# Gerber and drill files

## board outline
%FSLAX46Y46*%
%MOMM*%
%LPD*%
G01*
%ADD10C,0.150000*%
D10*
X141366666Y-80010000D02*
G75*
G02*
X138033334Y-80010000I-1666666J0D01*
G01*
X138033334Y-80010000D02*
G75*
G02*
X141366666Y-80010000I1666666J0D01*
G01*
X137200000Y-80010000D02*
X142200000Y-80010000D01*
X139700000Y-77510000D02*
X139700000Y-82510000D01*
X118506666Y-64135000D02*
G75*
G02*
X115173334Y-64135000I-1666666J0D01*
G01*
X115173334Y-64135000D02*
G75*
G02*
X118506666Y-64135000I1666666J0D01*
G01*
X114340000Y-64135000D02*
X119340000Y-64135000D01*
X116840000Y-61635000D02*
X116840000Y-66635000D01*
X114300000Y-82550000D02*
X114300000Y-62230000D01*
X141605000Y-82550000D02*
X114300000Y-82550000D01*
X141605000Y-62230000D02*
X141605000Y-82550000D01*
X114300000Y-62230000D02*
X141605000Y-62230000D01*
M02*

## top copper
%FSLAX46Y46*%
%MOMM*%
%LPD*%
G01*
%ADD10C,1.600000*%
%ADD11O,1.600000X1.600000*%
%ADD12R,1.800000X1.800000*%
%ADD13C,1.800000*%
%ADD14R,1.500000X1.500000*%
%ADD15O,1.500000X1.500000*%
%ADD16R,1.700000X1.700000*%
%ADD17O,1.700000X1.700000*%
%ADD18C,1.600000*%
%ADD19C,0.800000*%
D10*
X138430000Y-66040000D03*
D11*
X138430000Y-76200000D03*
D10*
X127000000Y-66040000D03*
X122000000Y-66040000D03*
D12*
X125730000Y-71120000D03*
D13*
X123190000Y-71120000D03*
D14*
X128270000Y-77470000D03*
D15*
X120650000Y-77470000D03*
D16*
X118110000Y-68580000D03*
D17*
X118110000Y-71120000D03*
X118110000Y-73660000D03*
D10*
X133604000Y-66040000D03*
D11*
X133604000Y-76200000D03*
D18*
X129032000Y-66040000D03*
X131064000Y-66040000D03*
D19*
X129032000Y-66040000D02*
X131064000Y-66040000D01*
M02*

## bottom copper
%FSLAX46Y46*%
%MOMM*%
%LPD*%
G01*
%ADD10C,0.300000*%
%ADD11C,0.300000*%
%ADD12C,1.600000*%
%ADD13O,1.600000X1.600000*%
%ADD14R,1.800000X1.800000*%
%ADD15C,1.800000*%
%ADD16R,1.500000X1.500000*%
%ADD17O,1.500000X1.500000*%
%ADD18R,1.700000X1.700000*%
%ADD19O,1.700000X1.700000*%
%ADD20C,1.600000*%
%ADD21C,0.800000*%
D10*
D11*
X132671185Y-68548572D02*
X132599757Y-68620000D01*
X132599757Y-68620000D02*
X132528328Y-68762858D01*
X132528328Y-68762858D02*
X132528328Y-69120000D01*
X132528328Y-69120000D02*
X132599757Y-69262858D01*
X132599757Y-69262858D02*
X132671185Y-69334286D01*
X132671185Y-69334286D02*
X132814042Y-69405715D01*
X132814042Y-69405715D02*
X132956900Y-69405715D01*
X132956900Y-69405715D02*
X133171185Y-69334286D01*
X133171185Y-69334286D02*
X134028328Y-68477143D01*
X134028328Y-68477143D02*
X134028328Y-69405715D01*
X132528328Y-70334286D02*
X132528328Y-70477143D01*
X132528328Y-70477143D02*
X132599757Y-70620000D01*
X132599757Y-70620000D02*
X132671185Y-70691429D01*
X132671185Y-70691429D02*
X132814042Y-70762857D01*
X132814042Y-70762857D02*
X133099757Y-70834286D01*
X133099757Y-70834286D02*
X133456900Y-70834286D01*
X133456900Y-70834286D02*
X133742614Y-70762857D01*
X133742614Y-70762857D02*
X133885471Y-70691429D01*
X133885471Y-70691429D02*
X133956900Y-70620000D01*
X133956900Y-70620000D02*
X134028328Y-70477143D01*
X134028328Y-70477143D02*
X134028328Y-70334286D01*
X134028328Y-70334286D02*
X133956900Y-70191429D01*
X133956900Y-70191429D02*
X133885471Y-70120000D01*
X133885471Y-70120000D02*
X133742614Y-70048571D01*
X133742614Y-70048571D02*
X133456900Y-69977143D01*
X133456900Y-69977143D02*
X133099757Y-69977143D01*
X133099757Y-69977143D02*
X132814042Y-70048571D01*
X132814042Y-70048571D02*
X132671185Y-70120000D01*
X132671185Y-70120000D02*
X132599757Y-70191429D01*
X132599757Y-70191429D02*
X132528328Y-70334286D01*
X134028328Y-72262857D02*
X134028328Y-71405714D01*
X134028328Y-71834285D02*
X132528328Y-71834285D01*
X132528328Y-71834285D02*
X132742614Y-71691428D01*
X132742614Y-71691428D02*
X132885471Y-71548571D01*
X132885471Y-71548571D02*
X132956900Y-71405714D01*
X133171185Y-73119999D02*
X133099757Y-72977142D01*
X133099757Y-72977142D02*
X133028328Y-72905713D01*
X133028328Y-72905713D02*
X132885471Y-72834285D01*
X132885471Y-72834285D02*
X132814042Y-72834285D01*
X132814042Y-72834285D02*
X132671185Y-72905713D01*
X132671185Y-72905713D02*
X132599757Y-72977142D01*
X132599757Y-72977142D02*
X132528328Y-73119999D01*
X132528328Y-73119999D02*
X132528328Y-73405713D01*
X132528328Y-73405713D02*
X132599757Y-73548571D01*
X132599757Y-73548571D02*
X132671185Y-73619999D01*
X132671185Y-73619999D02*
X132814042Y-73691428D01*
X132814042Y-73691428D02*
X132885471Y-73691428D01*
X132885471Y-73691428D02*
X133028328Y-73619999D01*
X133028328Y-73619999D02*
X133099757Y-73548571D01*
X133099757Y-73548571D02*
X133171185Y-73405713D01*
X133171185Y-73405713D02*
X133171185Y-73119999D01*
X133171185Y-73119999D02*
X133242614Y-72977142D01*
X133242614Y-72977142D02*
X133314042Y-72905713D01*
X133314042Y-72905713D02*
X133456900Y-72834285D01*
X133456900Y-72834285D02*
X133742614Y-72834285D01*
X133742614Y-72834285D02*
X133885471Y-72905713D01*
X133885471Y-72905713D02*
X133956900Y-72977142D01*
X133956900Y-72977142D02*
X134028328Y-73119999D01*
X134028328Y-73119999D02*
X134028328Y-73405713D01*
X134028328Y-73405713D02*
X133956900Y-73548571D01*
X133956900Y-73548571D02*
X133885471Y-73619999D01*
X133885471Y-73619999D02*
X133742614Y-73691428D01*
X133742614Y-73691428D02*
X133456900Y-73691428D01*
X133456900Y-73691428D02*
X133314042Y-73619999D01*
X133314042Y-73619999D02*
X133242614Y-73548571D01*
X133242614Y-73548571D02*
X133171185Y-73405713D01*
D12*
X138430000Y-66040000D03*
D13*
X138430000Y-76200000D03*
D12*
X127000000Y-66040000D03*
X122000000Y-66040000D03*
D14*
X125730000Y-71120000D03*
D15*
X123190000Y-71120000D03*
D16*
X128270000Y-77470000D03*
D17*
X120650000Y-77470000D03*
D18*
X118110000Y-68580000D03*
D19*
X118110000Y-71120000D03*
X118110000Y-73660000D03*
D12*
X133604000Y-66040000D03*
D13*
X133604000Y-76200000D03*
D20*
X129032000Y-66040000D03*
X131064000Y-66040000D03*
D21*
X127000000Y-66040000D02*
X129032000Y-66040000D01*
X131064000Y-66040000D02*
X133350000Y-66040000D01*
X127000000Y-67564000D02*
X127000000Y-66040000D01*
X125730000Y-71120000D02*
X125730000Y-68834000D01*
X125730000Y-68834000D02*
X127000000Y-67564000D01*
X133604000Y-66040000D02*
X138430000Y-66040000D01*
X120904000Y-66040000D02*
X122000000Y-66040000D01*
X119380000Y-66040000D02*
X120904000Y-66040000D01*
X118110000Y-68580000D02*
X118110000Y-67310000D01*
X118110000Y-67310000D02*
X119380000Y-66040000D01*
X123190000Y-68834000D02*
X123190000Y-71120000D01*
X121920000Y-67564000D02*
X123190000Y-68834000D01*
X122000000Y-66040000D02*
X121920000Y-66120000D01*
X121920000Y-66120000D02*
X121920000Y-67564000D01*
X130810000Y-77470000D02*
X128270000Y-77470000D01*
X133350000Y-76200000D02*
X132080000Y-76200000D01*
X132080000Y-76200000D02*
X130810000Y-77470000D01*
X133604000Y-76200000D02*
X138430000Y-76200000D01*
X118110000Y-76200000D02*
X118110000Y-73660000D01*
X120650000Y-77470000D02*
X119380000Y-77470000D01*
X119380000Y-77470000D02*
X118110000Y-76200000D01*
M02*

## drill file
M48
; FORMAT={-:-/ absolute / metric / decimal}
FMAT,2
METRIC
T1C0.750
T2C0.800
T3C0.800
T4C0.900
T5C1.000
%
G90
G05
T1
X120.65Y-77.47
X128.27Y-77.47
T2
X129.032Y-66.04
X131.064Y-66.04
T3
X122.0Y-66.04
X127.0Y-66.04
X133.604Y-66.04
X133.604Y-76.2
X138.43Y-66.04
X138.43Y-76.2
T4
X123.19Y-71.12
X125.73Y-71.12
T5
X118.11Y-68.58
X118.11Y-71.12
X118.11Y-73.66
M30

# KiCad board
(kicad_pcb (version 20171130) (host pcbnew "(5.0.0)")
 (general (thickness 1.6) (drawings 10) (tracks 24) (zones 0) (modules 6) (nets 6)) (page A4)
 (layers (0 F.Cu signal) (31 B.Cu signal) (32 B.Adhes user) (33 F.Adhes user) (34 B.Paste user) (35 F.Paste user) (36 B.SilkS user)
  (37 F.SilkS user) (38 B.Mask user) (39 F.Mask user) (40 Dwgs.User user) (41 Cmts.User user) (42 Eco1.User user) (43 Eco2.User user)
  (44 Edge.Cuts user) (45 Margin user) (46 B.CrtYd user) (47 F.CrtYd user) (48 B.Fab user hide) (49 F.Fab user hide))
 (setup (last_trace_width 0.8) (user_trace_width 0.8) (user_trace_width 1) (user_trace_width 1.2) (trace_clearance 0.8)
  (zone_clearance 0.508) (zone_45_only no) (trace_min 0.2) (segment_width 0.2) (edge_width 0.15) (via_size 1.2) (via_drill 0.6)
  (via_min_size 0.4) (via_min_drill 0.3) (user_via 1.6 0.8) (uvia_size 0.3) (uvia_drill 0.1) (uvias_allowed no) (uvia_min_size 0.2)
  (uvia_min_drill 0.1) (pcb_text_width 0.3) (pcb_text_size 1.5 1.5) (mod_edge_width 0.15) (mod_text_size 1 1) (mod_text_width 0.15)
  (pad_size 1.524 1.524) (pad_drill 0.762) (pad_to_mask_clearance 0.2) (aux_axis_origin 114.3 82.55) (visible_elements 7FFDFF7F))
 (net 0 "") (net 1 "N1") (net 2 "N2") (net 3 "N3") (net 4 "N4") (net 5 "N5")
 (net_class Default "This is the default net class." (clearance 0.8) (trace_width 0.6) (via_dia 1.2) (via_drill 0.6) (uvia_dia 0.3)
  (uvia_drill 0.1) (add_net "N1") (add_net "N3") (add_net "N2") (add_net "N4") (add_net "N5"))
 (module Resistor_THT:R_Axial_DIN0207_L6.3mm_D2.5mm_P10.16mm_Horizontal (layer F.Cu) (at 138.43 66.04 270)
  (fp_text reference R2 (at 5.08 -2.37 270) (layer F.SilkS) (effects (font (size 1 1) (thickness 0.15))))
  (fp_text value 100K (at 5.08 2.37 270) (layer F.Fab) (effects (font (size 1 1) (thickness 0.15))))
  (pad 1 thru_hole circle (at 0 0 270) (size 1.6 1.6) (drill 0.8) (layers *.Cu *.Mask) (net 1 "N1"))
  (pad 2 thru_hole oval (at 10.16 0 270) (size 1.6 1.6) (drill 0.8) (layers *.Cu *.Mask) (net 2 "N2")))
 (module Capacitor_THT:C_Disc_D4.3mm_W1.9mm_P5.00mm (layer F.Cu) (at 127 66.04 180)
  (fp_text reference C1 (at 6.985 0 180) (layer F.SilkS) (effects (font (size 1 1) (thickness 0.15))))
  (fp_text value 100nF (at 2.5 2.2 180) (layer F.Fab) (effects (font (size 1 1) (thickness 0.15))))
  (pad 1 thru_hole circle (at 0 0 180) (size 1.6 1.6) (drill 0.8) (layers *.Cu *.Mask) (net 1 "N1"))
  (pad 2 thru_hole circle (at 5 0 180) (size 1.6 1.6) (drill 0.8) (layers *.Cu *.Mask) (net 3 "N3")))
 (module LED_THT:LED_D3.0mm (layer F.Cu) (at 125.73 71.12 180) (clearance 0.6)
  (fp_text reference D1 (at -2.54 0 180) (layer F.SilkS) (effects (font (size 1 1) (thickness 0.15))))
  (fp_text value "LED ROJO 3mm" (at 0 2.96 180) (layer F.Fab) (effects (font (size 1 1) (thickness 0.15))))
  (pad 1 thru_hole rect (at 0 0 180) (size 1.8 1.8) (drill 0.9) (layers *.Cu *.Mask) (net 1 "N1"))
  (pad 2 thru_hole circle (at 2.54 0 180) (size 1.8 1.8) (drill 0.9) (layers *.Cu *.Mask) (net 3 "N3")))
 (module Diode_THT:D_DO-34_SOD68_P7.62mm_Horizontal (layer F.Cu) (at 128.27 77.47 180)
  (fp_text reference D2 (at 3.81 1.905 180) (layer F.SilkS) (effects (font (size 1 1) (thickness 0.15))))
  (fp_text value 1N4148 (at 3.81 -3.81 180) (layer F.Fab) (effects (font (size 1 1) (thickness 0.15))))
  (pad 1 thru_hole rect (at 0 0 180) (size 1.5 1.5) (drill 0.75) (layers *.Cu *.Mask) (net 2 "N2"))
  (pad 2 thru_hole oval (at 7.62 0 180) (size 1.5 1.5) (drill 0.75) (layers *.Cu *.Mask) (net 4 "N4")))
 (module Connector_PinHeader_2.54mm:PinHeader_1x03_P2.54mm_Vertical (layer F.Cu) (at 118.11 68.58)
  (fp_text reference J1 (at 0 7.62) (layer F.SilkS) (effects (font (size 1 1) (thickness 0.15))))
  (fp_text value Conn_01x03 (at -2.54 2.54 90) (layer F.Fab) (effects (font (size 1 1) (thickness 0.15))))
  (pad 1 thru_hole rect (at 0 0) (size 1.7 1.7) (drill 1) (layers *.Cu *.Mask) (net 3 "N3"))
  (pad 2 thru_hole oval (at 0 2.54) (size 1.7 1.7) (drill 1) (layers *.Cu *.Mask) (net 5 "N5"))
  (pad 3 thru_hole oval (at 0 5.08) (size 1.7 1.7) (drill 1) (layers *.Cu *.Mask) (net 4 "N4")))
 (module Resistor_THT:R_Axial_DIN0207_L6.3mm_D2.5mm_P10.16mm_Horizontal (layer F.Cu) (at 133.604 66.04 270)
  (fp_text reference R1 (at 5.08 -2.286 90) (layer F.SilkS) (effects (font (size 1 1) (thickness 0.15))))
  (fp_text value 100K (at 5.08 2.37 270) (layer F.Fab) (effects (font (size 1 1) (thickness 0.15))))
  (pad 1 thru_hole circle (at 0 0 270) (size 1.6 1.6) (drill 0.8) (layers *.Cu *.Mask) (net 1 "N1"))
  (pad 2 thru_hole oval (at 10.16 0 270) (size 1.6 1.6) (drill 0.8) (layers *.Cu *.Mask) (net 2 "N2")))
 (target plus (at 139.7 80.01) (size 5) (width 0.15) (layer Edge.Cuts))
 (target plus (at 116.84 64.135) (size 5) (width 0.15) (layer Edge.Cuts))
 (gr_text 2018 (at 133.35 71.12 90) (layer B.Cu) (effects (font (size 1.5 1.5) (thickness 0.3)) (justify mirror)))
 (gr_line (start 114.3 82.55) (end 114.3 62.23) (layer Edge.Cuts) (width 0.15))
 (gr_line (start 141.605 82.55) (end 114.3 82.55) (layer Edge.Cuts) (width 0.15))
 (gr_line (start 141.605 62.23) (end 141.605 82.55) (layer Edge.Cuts) (width 0.15))
 (gr_line (start 114.3 62.23) (end 141.605 62.23) (layer Edge.Cuts) (width 0.15))
 (via (at 129.032 66.04) (size 1.6) (drill 0.8) (layers F.Cu B.Cu) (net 1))
 (segment (start 127 66.04) (end 129.032 66.04) (width 0.8) (layer B.Cu) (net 1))
 (segment (start 129.032 66.04) (end 131.064 66.04) (width 0.8) (layer F.Cu) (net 1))
 (via (at 131.064 66.04) (size 1.6) (drill 0.8) (layers F.Cu B.Cu) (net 1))
 (segment (start 131.064 66.04) (end 133.35 66.04) (width 0.8) (layer B.Cu) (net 1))
 (segment (start 127 67.564) (end 127 66.04) (width 0.8) (layer B.Cu) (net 1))
 (segment (start 125.73 71.12) (end 125.73 68.834) (width 0.8) (layer B.Cu) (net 1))
 (segment (start 125.73 68.834) (end 127 67.564) (width 0.8) (layer B.Cu) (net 1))
 (segment (start 133.604 66.04) (end 138.43 66.04) (width 0.8) (layer B.Cu) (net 1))
 (segment (start 120.904 66.04) (end 122 66.04) (width 0.8) (layer B.Cu) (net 3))
 (segment (start 119.38 66.04) (end 120.904 66.04) (width 0.8) (layer B.Cu) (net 3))
 (segment (start 118.11 68.58) (end 118.11 67.31) (width 0.8) (layer B.Cu) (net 3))
 (segment (start 118.11 67.31) (end 119.38 66.04) (width 0.8) (layer B.Cu) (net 3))
 (segment (start 123.19 68.834) (end 123.19 71.12) (width 0.8) (layer B.Cu) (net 3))
 (segment (start 121.92 67.564) (end 123.19 68.834) (width 0.8) (layer B.Cu) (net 3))
 (segment (start 122 66.04) (end 121.92 66.12) (width 0.8) (layer B.Cu) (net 3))
 (segment (start 121.92 66.12) (end 121.92 67.564) (width 0.8) (layer B.Cu) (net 3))
 (segment (start 130.81 77.47) (end 128.27 77.47) (width 0.8) (layer B.Cu) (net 2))
 (segment (start 133.35 76.2) (end 132.08 76.2) (width 0.8) (layer B.Cu) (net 2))
 (segment (start 132.08 76.2) (end 130.81 77.47) (width 0.8) (layer B.Cu) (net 2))
 (segment (start 133.604 76.2) (end 138.43 76.2) (width 0.8) (layer B.Cu) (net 2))
 (segment (start 118.11 76.2) (end 118.11 73.66) (width 0.8) (layer B.Cu) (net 4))
 (segment (start 120.65 77.47) (end 119.38 77.47) (width 0.8) (layer B.Cu) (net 4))
 (segment (start 119.38 77.47) (end 118.11 76.2) (width 0.8) (layer B.Cu) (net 4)))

